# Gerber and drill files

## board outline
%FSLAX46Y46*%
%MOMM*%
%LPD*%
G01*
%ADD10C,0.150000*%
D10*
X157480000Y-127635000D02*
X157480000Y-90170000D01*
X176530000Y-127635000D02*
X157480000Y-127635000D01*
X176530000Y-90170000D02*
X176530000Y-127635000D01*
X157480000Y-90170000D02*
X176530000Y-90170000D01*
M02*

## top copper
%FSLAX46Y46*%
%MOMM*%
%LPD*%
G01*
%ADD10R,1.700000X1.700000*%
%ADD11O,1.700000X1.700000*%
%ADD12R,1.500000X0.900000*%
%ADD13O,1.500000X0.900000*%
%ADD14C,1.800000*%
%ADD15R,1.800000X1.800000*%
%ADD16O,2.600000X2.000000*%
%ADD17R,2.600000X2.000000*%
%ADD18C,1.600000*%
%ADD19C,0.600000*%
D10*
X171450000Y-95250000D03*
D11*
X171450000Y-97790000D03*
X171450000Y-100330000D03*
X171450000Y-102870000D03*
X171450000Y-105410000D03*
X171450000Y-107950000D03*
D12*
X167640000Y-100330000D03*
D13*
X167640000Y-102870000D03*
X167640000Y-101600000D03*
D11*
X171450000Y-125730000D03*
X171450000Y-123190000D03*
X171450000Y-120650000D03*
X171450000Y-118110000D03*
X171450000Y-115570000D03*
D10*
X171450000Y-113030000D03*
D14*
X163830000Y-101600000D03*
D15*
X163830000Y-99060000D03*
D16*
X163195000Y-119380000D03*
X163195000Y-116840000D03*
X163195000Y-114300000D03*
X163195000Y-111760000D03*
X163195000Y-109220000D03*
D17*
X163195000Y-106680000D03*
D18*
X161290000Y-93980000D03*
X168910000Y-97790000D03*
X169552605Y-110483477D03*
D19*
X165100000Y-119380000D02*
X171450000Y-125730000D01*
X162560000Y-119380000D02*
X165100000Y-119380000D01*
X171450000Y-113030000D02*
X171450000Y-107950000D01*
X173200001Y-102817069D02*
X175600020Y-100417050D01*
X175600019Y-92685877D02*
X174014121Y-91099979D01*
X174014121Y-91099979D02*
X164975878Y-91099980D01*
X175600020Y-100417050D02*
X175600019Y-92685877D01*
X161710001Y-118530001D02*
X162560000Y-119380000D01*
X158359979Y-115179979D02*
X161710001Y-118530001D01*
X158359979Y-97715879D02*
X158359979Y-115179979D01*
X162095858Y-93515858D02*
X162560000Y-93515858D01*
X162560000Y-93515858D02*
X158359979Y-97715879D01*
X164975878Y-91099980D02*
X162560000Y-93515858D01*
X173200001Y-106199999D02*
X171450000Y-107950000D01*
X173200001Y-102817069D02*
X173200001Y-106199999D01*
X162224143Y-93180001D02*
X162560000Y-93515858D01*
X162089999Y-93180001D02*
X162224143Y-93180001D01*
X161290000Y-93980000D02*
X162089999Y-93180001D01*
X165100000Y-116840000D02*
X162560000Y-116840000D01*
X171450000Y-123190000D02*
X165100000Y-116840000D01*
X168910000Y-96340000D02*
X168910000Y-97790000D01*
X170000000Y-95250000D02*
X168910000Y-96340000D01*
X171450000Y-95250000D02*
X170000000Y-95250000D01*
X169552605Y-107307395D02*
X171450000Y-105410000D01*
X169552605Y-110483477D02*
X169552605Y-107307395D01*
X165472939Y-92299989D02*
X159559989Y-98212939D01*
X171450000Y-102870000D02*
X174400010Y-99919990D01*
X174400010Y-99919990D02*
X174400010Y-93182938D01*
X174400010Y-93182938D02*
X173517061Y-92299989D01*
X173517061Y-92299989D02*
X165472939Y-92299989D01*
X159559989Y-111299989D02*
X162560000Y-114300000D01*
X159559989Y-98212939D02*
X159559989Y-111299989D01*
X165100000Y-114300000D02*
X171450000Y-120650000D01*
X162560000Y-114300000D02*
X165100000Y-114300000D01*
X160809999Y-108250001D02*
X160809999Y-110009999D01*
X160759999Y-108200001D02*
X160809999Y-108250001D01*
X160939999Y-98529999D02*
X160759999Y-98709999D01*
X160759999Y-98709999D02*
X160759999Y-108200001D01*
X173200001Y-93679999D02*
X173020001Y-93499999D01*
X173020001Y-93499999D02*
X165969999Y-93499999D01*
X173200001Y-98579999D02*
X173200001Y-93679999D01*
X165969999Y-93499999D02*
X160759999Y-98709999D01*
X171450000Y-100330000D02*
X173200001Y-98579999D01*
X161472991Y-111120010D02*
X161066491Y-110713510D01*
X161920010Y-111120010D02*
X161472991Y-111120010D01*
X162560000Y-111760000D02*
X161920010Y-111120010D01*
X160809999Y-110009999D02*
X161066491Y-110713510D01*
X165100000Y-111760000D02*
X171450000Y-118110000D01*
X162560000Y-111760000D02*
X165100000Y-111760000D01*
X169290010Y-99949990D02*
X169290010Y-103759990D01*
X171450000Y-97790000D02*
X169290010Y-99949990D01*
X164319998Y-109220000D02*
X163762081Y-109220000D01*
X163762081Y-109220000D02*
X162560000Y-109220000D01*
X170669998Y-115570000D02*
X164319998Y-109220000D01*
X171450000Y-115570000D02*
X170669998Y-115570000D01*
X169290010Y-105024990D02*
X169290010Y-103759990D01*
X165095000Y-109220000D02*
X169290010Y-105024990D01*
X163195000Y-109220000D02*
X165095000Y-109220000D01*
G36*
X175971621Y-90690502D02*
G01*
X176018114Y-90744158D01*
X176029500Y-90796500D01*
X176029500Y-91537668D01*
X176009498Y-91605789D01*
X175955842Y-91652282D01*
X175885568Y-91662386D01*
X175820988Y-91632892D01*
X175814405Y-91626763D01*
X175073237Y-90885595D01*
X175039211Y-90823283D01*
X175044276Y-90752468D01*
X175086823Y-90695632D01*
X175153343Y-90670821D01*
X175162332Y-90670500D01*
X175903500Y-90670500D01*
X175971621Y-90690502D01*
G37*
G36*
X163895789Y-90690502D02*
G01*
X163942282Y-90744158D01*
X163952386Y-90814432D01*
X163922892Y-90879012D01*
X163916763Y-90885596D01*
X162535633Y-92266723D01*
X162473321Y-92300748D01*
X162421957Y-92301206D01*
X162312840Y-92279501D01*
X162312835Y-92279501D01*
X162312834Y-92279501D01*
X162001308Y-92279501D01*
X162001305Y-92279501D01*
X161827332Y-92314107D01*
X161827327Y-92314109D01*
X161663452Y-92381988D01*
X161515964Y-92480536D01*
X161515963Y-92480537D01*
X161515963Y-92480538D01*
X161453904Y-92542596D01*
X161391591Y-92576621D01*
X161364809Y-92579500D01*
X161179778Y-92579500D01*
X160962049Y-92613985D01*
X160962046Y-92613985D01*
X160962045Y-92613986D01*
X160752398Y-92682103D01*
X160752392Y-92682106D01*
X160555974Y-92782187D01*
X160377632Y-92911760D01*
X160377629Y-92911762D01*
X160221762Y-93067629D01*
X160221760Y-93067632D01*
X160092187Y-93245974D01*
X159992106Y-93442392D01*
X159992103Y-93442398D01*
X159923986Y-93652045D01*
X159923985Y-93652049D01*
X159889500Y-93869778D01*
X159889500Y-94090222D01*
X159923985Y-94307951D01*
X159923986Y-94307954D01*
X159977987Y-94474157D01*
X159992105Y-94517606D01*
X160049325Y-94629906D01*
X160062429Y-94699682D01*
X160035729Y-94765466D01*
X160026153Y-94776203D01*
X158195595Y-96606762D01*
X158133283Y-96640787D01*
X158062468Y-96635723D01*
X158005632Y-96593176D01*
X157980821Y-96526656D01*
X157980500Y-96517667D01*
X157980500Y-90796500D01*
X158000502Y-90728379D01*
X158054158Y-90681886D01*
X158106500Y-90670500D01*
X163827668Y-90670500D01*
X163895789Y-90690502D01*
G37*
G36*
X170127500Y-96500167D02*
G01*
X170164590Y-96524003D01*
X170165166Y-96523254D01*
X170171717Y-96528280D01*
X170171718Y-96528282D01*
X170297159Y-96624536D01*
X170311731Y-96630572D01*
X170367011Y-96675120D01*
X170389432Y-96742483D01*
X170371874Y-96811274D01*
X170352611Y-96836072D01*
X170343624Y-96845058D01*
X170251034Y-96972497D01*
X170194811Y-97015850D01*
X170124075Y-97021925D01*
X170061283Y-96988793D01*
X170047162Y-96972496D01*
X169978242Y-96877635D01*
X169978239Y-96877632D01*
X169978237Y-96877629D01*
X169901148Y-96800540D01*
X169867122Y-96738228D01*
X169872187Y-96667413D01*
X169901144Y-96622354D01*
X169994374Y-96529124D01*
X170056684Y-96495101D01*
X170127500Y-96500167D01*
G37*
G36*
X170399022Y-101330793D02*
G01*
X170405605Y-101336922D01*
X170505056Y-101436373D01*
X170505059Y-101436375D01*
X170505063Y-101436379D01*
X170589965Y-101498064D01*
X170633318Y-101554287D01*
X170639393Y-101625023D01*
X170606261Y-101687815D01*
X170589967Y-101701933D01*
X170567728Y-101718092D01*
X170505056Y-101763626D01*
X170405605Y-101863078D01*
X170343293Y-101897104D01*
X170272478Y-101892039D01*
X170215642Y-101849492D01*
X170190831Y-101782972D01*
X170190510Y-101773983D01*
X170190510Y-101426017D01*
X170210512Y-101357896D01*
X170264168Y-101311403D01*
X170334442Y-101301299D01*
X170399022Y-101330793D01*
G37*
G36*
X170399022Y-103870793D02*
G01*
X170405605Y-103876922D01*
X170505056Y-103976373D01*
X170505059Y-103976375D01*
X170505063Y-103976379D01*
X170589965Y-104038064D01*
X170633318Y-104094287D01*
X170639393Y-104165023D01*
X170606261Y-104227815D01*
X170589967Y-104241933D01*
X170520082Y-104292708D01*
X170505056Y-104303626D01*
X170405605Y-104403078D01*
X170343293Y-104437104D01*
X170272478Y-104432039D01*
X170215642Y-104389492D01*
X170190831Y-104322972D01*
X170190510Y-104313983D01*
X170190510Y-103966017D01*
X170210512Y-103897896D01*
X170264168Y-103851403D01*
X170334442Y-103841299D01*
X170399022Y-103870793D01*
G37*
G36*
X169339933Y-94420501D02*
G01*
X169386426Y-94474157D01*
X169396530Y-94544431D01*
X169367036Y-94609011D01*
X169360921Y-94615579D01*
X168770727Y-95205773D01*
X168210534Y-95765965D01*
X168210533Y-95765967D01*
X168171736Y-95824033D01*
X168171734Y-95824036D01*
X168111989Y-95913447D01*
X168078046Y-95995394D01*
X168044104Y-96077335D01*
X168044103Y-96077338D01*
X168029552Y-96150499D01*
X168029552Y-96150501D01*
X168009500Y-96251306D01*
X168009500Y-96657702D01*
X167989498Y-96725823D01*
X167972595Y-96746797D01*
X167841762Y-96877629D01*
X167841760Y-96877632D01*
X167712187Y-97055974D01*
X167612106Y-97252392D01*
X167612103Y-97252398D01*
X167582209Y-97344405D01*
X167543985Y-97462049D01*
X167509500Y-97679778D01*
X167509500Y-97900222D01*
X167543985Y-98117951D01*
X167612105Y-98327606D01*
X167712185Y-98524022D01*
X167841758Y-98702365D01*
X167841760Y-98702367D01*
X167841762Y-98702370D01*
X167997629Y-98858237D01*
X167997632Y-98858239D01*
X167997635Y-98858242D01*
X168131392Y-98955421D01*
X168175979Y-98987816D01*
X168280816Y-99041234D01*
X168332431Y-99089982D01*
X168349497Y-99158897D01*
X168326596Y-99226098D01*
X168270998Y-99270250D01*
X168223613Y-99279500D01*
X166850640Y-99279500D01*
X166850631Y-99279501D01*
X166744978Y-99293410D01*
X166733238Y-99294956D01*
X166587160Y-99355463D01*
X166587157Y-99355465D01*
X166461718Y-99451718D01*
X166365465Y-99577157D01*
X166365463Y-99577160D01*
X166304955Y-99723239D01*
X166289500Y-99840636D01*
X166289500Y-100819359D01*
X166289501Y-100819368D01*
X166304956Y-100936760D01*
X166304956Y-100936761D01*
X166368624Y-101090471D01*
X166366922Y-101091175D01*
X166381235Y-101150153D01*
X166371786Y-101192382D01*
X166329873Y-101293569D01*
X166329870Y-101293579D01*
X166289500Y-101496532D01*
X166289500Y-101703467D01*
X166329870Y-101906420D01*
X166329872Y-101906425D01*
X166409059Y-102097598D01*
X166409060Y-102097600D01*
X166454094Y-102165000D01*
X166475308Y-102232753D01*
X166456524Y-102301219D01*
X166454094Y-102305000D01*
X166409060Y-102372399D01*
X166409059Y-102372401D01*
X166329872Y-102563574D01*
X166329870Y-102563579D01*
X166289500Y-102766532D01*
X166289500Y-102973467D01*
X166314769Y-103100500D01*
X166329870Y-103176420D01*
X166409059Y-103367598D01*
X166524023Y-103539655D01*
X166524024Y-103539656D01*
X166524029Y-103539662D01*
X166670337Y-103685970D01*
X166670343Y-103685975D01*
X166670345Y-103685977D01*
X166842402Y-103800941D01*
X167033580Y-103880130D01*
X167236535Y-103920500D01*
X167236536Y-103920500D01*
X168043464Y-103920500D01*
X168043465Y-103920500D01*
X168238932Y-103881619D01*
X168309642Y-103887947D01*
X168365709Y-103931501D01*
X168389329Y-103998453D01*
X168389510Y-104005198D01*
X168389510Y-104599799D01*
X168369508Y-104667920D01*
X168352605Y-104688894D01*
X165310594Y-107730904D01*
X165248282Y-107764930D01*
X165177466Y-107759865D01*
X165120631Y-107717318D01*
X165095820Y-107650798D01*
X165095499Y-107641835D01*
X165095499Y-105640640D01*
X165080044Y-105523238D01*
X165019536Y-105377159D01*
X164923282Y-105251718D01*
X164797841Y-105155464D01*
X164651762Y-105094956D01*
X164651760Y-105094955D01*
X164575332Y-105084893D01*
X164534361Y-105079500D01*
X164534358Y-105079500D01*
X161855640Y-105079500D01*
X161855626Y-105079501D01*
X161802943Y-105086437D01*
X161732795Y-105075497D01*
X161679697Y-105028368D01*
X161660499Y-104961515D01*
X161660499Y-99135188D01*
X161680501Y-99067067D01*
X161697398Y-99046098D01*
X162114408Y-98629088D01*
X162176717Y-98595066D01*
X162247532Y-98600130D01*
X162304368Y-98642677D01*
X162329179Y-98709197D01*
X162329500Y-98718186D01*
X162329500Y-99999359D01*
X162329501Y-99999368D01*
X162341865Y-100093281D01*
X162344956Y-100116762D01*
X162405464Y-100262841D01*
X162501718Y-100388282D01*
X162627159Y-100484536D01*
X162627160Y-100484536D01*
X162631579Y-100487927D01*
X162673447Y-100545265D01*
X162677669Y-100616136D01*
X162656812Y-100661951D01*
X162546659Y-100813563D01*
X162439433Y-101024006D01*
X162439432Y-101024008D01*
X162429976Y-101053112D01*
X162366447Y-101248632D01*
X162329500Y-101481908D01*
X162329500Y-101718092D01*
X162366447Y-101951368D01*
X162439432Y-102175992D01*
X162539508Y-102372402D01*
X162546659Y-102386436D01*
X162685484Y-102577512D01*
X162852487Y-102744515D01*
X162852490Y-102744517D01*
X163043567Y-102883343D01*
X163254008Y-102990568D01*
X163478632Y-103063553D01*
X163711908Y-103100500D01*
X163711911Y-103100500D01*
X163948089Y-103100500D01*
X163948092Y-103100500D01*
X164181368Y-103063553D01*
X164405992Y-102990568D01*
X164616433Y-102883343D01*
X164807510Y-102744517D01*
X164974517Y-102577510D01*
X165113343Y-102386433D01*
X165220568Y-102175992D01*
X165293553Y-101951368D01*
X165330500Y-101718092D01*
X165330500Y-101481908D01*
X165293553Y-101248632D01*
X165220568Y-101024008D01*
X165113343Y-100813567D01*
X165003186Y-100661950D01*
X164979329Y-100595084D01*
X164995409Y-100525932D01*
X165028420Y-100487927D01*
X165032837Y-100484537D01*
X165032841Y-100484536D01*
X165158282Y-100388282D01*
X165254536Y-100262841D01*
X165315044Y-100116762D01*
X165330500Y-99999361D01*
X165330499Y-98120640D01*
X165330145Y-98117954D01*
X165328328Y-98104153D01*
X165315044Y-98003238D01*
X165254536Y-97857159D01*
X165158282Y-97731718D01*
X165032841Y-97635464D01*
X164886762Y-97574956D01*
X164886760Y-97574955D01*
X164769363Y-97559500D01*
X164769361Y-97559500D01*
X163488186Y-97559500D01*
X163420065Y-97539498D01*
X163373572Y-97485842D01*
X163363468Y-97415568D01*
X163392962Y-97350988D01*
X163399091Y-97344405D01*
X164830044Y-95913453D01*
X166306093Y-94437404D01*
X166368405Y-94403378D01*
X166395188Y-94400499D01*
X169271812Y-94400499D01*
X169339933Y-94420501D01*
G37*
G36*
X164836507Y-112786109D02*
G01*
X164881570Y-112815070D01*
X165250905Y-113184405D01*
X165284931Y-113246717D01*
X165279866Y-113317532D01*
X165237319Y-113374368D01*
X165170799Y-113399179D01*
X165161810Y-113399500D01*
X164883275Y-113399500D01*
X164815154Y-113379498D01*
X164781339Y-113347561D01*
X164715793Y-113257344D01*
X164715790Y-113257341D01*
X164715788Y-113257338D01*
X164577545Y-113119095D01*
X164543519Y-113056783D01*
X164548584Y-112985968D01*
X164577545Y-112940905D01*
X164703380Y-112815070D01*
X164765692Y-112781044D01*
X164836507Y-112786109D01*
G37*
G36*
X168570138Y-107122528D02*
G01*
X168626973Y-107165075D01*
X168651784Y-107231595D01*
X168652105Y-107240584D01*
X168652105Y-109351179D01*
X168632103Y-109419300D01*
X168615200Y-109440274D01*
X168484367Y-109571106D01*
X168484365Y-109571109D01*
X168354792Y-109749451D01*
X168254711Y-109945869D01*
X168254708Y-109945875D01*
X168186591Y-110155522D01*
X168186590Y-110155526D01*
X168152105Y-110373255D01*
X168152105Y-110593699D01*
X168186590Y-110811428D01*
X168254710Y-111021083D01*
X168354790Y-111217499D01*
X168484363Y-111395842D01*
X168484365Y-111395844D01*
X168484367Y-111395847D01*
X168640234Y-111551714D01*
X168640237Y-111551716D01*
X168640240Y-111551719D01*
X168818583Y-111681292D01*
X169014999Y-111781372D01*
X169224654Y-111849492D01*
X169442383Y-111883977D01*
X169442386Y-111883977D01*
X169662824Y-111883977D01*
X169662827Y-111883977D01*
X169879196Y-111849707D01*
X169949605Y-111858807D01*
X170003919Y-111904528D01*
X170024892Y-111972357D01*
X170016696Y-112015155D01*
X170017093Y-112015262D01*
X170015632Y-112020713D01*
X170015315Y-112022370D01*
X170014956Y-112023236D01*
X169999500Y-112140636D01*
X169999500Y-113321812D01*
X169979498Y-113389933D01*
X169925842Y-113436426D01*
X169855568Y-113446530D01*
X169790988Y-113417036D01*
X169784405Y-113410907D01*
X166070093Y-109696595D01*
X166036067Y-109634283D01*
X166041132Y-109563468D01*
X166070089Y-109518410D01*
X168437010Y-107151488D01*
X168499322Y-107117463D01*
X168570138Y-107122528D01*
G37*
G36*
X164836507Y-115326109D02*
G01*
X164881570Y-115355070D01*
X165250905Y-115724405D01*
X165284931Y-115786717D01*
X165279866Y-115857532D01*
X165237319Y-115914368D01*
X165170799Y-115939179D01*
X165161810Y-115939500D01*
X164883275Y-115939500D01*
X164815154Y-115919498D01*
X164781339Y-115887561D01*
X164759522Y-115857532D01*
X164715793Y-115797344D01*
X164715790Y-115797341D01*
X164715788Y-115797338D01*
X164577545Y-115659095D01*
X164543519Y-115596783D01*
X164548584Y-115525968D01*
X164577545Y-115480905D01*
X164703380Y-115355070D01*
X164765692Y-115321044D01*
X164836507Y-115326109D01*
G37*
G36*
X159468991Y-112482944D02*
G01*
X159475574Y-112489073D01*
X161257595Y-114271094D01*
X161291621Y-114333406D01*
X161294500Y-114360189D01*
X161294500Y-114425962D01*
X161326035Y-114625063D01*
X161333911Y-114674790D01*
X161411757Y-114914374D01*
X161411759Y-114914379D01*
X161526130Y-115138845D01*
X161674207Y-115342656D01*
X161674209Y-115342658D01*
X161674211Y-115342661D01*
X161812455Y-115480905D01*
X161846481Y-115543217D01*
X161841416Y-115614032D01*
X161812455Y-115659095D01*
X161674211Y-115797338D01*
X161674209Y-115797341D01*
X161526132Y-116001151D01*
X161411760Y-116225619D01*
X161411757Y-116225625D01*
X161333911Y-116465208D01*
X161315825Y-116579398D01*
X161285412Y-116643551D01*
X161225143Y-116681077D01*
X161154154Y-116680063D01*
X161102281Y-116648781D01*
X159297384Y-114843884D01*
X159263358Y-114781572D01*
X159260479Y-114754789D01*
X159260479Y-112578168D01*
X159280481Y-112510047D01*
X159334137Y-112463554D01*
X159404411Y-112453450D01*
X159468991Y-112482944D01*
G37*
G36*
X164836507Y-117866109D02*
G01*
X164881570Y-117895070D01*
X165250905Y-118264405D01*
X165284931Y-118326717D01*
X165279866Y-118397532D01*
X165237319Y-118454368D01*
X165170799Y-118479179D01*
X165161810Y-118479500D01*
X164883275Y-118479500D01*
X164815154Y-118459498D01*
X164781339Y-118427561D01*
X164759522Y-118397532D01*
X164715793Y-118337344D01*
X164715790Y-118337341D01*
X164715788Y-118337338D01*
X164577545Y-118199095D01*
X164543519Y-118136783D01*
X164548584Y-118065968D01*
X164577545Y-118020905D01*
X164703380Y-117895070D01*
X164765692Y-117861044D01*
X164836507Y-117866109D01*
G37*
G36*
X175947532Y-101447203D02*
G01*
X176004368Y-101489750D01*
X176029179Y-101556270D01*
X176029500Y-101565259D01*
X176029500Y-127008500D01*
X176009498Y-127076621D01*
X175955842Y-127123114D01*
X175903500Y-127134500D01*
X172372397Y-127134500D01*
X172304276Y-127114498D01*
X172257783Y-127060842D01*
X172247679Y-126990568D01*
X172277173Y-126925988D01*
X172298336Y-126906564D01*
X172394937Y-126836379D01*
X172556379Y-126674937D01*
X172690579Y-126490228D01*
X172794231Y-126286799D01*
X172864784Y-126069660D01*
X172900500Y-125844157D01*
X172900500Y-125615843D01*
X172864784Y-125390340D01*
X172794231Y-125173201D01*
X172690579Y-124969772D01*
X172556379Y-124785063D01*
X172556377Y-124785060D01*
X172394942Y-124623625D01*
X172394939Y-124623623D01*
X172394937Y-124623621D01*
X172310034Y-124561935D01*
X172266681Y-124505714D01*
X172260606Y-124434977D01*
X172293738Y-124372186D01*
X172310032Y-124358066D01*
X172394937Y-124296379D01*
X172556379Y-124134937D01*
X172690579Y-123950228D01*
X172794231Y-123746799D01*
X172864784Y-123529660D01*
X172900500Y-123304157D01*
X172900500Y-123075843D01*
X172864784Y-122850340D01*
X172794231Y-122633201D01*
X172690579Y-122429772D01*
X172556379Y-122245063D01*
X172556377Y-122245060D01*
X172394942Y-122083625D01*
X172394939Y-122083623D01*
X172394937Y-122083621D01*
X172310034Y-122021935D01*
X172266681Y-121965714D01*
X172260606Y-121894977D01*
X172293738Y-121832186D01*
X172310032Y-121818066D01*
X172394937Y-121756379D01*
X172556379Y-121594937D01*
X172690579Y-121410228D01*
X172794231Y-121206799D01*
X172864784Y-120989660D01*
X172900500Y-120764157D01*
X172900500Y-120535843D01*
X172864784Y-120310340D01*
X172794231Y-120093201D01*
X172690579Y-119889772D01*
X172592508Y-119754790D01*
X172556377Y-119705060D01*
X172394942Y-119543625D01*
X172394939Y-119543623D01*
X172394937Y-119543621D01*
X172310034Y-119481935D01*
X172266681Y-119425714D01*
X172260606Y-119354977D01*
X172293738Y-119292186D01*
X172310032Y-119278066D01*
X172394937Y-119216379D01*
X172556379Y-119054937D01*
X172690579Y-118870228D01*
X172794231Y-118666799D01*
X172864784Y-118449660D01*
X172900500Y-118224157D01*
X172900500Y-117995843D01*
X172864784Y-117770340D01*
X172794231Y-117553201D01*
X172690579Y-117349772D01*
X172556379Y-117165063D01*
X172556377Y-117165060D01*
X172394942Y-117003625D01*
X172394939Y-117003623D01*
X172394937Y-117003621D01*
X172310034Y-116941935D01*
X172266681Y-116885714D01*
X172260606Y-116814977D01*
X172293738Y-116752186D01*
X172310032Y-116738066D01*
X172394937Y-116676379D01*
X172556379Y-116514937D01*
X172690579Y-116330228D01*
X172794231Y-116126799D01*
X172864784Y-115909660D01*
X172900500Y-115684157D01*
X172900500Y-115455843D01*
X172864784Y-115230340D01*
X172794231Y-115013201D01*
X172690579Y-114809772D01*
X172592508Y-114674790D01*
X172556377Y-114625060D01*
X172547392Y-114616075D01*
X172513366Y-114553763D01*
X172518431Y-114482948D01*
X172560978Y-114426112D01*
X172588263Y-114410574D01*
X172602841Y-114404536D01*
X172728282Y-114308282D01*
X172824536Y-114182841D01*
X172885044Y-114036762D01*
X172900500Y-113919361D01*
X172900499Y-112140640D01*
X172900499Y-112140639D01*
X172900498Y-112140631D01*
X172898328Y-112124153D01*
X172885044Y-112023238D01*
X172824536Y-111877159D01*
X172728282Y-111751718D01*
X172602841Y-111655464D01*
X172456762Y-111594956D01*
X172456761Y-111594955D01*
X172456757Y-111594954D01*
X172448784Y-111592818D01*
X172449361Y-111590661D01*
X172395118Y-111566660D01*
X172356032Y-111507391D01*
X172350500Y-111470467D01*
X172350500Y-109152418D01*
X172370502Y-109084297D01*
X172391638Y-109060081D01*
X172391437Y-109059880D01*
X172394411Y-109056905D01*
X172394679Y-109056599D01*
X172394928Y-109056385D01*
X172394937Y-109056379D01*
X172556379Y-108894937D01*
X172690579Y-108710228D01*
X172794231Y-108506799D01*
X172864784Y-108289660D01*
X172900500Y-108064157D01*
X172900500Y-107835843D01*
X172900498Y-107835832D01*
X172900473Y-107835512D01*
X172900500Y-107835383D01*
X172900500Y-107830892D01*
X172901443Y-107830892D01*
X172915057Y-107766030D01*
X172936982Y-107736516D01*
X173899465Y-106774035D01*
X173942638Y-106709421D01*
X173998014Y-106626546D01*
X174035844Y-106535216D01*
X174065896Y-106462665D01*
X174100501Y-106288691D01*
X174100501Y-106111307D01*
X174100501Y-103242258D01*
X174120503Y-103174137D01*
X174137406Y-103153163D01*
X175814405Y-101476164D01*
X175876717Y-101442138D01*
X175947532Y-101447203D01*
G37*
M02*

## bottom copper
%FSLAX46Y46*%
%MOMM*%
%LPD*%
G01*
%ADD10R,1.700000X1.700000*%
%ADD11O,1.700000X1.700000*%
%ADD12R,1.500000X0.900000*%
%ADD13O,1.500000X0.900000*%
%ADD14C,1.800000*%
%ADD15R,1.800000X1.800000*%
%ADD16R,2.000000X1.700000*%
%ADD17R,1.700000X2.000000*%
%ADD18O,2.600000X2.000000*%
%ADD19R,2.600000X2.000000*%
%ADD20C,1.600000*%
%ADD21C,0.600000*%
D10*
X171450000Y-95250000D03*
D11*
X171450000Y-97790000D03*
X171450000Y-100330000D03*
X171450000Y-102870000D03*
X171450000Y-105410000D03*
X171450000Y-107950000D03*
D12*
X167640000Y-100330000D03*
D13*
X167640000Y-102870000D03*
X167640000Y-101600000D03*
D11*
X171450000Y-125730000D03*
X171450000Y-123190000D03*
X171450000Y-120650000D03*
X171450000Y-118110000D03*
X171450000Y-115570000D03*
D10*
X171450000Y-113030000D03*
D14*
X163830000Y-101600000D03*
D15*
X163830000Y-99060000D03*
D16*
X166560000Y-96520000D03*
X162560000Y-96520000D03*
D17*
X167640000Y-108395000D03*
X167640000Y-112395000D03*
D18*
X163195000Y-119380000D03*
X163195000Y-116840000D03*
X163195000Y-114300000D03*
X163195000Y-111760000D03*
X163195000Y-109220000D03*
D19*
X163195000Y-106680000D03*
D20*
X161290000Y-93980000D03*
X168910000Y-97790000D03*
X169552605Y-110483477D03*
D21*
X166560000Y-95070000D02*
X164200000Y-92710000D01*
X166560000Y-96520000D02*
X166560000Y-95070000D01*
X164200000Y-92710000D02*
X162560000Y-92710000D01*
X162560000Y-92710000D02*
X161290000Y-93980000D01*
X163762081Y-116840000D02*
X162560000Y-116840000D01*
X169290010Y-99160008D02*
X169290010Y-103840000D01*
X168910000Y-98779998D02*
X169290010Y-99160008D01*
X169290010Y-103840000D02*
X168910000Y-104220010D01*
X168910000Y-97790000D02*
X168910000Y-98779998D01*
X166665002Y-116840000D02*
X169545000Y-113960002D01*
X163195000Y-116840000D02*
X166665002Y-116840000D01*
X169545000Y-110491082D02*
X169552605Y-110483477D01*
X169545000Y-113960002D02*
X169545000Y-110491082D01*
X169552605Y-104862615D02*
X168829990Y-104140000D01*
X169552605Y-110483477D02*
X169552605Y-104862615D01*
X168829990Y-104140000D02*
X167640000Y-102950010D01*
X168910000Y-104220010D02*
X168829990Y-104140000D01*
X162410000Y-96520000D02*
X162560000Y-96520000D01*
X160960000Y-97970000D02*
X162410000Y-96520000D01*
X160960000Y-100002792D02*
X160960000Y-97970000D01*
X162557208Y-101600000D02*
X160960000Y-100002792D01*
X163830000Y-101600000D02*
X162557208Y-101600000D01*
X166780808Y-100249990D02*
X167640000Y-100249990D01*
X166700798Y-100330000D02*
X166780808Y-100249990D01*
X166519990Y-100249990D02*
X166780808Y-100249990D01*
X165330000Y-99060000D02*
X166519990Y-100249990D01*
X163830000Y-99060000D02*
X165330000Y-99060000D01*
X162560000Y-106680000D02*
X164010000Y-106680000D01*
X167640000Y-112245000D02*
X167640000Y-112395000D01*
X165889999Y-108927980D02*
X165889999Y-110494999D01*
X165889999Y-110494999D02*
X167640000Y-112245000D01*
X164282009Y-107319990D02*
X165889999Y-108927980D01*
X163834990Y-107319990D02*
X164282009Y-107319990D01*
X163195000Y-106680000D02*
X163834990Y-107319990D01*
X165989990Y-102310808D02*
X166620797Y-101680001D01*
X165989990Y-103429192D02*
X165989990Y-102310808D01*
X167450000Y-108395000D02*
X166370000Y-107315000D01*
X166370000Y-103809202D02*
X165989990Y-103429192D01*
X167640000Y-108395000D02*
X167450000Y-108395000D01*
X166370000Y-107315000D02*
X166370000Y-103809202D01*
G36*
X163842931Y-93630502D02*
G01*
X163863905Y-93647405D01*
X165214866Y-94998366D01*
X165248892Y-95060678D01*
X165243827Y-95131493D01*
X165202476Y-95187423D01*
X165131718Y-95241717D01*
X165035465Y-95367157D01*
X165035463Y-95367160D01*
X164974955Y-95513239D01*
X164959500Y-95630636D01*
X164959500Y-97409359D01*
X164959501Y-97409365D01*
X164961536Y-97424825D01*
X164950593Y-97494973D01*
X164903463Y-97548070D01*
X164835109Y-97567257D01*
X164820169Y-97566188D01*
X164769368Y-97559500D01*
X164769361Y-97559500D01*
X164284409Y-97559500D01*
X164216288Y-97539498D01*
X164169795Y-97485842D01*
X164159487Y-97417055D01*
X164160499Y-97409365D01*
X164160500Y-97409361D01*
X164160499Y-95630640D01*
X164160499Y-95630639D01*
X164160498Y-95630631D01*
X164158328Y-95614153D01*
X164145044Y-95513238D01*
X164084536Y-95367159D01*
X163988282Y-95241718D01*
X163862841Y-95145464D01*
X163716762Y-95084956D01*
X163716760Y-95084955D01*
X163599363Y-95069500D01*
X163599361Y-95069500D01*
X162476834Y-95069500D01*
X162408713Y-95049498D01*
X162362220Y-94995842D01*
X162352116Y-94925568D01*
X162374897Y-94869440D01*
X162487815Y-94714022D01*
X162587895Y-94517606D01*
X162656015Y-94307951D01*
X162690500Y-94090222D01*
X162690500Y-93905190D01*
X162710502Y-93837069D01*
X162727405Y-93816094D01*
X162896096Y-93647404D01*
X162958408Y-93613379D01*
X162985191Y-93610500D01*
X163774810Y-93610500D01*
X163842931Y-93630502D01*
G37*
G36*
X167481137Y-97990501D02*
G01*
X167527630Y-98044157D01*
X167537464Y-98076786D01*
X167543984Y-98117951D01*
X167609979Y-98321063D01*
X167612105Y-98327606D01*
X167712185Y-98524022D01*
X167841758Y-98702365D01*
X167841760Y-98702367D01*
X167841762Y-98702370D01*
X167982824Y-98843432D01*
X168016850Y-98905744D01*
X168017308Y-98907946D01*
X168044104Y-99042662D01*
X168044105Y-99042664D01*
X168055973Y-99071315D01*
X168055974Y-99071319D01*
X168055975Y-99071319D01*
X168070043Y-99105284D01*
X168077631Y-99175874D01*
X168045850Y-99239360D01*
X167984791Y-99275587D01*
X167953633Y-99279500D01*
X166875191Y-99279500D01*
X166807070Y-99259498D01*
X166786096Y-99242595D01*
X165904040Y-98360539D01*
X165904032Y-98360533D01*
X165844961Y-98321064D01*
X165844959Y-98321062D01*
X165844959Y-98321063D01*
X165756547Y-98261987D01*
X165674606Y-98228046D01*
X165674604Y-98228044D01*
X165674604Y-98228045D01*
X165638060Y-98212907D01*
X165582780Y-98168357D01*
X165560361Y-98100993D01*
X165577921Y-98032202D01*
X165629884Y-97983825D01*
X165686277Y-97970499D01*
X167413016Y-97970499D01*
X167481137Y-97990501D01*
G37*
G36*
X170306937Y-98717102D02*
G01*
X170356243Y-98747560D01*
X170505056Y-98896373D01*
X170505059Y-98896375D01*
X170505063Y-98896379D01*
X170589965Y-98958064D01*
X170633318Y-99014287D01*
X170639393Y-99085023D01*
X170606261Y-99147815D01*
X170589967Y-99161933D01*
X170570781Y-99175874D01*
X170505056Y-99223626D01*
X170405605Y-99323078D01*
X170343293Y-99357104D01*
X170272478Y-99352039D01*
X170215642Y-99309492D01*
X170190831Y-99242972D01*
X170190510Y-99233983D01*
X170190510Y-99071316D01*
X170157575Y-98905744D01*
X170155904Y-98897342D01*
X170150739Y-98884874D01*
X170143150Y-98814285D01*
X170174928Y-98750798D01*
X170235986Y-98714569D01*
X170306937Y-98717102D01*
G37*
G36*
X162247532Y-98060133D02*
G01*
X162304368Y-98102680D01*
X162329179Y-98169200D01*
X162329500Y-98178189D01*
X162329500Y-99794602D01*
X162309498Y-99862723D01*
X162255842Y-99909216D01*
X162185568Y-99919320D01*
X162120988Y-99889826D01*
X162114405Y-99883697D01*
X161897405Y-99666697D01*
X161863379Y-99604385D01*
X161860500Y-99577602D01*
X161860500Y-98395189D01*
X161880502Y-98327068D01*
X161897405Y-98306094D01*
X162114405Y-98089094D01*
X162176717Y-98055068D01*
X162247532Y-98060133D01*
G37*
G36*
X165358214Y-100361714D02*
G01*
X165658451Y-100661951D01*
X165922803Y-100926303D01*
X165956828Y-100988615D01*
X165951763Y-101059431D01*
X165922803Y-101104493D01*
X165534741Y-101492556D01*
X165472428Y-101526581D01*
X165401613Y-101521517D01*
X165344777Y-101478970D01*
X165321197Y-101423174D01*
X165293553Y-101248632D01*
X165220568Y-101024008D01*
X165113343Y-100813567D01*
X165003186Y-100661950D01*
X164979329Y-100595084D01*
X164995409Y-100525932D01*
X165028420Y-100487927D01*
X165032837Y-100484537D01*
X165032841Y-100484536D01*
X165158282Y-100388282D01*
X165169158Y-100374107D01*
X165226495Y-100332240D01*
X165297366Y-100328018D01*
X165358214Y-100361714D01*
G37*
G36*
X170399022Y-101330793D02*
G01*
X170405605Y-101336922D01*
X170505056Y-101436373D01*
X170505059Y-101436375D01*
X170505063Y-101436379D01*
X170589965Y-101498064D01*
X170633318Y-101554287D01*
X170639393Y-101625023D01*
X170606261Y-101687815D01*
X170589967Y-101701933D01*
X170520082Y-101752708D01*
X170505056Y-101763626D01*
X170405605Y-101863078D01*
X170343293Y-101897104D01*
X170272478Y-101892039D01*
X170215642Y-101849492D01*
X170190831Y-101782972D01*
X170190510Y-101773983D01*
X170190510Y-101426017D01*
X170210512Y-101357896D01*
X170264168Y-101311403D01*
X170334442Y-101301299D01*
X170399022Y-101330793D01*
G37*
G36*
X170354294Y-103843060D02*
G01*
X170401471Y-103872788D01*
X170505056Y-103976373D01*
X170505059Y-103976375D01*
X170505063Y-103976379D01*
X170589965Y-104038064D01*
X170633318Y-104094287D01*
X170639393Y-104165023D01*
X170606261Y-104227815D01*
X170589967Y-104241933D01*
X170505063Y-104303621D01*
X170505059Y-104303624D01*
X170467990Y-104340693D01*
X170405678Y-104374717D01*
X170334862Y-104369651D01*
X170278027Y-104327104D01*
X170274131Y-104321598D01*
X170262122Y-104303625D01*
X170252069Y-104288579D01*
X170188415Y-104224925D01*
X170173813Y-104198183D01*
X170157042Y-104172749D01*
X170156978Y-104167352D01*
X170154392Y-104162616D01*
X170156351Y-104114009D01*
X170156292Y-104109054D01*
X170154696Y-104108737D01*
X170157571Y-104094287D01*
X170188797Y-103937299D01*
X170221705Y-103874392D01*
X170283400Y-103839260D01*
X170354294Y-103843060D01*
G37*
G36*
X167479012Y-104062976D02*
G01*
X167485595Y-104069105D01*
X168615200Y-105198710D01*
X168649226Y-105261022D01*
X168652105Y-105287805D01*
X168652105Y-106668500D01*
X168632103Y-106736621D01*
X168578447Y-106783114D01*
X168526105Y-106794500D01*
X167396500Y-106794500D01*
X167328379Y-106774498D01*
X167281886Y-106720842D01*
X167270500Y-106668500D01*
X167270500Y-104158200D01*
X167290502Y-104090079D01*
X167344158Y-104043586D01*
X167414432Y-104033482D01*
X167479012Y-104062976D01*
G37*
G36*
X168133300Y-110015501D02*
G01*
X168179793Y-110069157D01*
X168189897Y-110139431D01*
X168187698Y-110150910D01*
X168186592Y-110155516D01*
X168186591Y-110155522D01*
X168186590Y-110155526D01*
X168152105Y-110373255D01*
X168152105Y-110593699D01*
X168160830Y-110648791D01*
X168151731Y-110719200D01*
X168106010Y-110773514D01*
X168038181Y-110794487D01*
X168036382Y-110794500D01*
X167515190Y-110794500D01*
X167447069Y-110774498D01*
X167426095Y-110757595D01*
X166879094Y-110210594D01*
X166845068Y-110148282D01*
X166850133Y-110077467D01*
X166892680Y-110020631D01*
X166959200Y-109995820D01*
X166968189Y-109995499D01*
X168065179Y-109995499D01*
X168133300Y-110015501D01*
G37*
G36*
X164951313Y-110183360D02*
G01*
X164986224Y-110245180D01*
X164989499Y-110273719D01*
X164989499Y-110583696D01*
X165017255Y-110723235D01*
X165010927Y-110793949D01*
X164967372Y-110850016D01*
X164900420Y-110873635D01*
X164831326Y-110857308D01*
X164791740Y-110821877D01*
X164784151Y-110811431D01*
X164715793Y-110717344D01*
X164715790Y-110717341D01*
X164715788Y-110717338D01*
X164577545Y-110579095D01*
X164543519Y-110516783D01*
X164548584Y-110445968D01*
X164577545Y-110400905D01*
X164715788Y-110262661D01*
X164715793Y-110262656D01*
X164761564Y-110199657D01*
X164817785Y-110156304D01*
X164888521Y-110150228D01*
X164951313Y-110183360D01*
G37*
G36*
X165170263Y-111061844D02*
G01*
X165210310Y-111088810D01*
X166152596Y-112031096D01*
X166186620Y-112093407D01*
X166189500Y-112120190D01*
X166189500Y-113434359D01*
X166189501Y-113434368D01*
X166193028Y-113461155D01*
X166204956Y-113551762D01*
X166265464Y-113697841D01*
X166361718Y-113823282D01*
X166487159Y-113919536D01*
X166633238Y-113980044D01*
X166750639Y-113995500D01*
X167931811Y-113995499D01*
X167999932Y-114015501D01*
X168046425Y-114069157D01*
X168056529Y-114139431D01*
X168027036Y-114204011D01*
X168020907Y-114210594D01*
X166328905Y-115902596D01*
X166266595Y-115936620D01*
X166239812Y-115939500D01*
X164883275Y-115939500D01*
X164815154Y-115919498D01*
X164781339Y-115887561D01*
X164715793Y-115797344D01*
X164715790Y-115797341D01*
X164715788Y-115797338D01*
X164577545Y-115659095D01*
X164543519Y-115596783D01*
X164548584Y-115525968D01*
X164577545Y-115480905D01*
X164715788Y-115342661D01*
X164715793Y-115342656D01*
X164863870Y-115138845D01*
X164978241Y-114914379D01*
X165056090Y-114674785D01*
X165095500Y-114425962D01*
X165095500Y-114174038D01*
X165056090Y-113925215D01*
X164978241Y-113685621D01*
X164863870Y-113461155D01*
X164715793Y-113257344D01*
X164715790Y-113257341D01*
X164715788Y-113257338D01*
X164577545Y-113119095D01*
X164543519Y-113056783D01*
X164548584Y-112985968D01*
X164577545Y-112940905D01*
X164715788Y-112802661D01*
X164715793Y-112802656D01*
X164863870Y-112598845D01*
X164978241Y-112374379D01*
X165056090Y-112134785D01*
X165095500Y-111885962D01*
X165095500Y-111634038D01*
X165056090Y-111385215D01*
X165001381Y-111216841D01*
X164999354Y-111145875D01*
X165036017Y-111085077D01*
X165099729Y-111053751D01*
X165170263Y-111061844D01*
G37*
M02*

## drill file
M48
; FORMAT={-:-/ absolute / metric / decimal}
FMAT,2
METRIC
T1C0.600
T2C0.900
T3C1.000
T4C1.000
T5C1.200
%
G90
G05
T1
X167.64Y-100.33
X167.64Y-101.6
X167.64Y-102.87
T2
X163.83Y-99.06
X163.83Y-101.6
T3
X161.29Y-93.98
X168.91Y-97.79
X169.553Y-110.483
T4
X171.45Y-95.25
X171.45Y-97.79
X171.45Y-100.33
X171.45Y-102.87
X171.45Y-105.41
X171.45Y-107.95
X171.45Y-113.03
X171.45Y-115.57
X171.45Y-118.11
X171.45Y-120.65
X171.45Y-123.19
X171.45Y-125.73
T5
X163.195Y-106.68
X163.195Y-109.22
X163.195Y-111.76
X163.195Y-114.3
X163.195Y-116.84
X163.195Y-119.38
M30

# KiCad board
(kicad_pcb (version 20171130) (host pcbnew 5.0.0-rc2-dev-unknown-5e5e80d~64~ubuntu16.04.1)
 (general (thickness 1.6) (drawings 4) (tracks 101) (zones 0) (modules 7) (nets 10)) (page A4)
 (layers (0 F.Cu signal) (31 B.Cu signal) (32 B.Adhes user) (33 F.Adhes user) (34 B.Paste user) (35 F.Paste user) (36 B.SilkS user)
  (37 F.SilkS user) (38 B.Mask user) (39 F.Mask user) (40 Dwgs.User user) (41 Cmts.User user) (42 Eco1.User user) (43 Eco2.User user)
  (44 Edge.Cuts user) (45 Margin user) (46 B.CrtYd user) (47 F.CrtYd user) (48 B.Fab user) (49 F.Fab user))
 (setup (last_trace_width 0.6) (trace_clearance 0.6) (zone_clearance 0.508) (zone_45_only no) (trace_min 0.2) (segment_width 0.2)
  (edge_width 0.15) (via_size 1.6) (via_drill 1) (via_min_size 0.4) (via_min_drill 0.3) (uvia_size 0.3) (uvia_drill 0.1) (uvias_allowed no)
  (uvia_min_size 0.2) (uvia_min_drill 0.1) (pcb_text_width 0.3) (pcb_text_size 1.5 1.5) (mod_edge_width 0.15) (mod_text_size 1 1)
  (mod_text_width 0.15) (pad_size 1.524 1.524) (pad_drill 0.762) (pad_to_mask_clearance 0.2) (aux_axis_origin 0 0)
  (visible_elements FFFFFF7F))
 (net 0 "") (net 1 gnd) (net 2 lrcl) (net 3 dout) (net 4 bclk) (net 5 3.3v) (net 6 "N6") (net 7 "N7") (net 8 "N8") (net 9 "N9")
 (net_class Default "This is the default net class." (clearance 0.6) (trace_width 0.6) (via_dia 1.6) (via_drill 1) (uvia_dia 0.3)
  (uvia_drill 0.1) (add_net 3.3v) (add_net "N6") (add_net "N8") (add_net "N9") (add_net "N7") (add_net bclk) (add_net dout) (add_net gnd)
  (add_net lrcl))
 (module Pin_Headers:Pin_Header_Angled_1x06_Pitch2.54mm (layer F.Cu) (at 171.45 95.25)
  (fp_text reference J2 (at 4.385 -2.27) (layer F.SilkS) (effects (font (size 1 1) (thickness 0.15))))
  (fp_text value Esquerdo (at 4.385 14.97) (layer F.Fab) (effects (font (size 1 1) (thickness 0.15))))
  (pad 1 thru_hole rect (at 0 0) (size 1.7 1.7) (drill 1) (layers *.Cu *.Mask) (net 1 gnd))
  (pad 2 thru_hole oval (at 0 2.54) (size 1.7 1.7) (drill 1) (layers *.Cu *.Mask) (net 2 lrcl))
  (pad 3 thru_hole oval (at 0 5.08) (size 1.7 1.7) (drill 1) (layers *.Cu *.Mask) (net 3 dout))
  (pad 4 thru_hole oval (at 0 7.62) (size 1.7 1.7) (drill 1) (layers *.Cu *.Mask) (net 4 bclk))
  (pad 5 thru_hole oval (at 0 10.16) (size 1.7 1.7) (drill 1) (layers *.Cu *.Mask) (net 1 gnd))
  (pad 6 thru_hole oval (at 0 12.7) (size 1.7 1.7) (drill 1) (layers *.Cu *.Mask) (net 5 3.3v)))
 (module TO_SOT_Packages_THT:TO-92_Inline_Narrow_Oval (layer F.Cu) (at 167.64 100.33 270)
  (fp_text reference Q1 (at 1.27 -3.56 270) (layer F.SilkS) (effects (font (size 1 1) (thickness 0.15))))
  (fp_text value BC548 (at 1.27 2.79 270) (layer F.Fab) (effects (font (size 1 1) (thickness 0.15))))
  (pad 1 thru_hole rect (at 0 0 90) (size 0.9 1.5) (drill 0.6) (layers *.Cu *.Mask) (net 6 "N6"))
  (pad 3 thru_hole oval (at 2.54 0 90) (size 0.9 1.5) (drill 0.6) (layers *.Cu *.Mask) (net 1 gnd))
  (pad 2 thru_hole oval (at 1.27 0 90) (size 0.9 1.5) (drill 0.6) (layers *.Cu *.Mask) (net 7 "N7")))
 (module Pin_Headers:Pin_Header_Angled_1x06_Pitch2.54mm (layer F.Cu) (at 171.45 113.03)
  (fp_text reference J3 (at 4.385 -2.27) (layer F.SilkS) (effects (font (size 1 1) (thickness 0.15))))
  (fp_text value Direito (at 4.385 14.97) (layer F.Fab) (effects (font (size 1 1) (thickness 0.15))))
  (pad 6 thru_hole oval (at 0 12.7) (size 1.7 1.7) (drill 1) (layers *.Cu *.Mask) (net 5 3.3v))
  (pad 5 thru_hole oval (at 0 10.16) (size 1.7 1.7) (drill 1) (layers *.Cu *.Mask) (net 1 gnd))
  (pad 4 thru_hole oval (at 0 7.62) (size 1.7 1.7) (drill 1) (layers *.Cu *.Mask) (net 4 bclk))
  (pad 3 thru_hole oval (at 0 5.08) (size 1.7 1.7) (drill 1) (layers *.Cu *.Mask) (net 3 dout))
  (pad 2 thru_hole oval (at 0 2.54) (size 1.7 1.7) (drill 1) (layers *.Cu *.Mask) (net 2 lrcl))
  (pad 1 thru_hole rect (at 0 0) (size 1.7 1.7) (drill 1) (layers *.Cu *.Mask) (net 5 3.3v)))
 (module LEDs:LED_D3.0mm (layer F.Cu) (at 163.83 99.06 270)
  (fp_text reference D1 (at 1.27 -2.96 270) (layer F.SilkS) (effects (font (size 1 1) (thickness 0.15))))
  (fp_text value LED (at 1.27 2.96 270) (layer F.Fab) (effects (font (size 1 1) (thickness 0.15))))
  (pad 2 thru_hole circle (at 2.54 0 270) (size 1.8 1.8) (drill 0.9) (layers *.Cu *.Mask) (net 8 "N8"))
  (pad 1 thru_hole rect (at 0 0 270) (size 1.8 1.8) (drill 0.9) (layers *.Cu *.Mask) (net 6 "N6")))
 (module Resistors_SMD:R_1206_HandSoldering (layer B.Cu) (at 164.56 96.52)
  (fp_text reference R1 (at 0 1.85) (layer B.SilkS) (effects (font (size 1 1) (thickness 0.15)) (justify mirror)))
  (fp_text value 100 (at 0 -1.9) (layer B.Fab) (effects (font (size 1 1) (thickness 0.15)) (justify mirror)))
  (pad 2 smd rect (at 2 0) (size 2 1.7) (layers B.Cu B.Paste B.Mask) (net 5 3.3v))
  (pad 1 smd rect (at -2 0) (size 2 1.7) (layers B.Cu B.Paste B.Mask) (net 8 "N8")))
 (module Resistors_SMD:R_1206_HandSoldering (layer B.Cu) (at 167.64 110.395 270)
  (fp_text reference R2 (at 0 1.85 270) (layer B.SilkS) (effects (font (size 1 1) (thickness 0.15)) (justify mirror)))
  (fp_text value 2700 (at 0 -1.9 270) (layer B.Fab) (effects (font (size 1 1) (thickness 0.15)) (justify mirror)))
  (pad 1 smd rect (at -2 0 270) (size 2 1.7) (layers B.Cu B.Paste B.Mask) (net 7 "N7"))
  (pad 2 smd rect (at 2 0 270) (size 2 1.7) (layers B.Cu B.Paste B.Mask) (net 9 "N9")))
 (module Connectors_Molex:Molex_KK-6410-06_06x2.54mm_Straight (layer F.Cu) (at 163.195 106.68 270)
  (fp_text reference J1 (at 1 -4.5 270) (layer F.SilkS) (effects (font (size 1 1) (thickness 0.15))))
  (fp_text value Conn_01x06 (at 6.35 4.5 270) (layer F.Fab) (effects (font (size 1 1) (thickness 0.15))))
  (pad 6 thru_hole oval (at 12.7 0 270) (size 2 2.6) (drill 1.2) (layers *.Cu *.Mask) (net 5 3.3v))
  (pad 5 thru_hole oval (at 10.16 0 270) (size 2 2.6) (drill 1.2) (layers *.Cu *.Mask) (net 1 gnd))
  (pad 4 thru_hole oval (at 7.62 0 270) (size 2 2.6) (drill 1.2) (layers *.Cu *.Mask) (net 4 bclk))
  (pad 3 thru_hole oval (at 5.08 0 270) (size 2 2.6) (drill 1.2) (layers *.Cu *.Mask) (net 3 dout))
  (pad 2 thru_hole oval (at 2.54 0 270) (size 2 2.6) (drill 1.2) (layers *.Cu *.Mask) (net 2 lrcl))
  (pad 1 thru_hole rect (at 0 0 270) (size 2 2.6) (drill 1.2) (layers *.Cu *.Mask) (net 9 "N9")))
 (gr_line (start 157.48 127.635) (end 157.48 90.17) (layer Edge.Cuts) (width 0.15))
 (gr_line (start 176.53 127.635) (end 157.48 127.635) (layer Edge.Cuts) (width 0.15))
 (gr_line (start 176.53 90.17) (end 176.53 127.635) (layer Edge.Cuts) (width 0.15))
 (gr_line (start 157.48 90.17) (end 176.53 90.17) (layer Edge.Cuts) (width 0.15))
 (segment (start 165.1 119.38) (end 171.45 125.73) (width 0.6) (layer F.Cu) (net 5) (status 20))
 (segment (start 162.56 119.38) (end 165.1 119.38) (width 0.6) (layer F.Cu) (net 5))
 (segment (start 171.45 113.03) (end 171.45 107.95) (width 0.6) (layer F.Cu) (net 5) (status 30))
 (segment (start 173.200001 102.817069) (end 175.60002 100.41705) (width 0.6) (layer F.Cu) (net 5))
 (segment (start 175.600019 92.685877) (end 174.014121 91.099979) (width 0.6) (layer F.Cu) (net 5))
 (segment (start 174.014121 91.099979) (end 164.975878 91.09998) (width 0.6) (layer F.Cu) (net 5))
 (segment (start 175.60002 100.41705) (end 175.600019 92.685877) (width 0.6) (layer F.Cu) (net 5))
 (segment (start 161.710001 118.530001) (end 162.56 119.38) (width 0.6) (layer F.Cu) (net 5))
 (segment (start 158.359979 115.179979) (end 161.710001 118.530001) (width 0.6) (layer F.Cu) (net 5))
 (segment (start 158.359979 97.715879) (end 158.359979 115.179979) (width 0.6) (layer F.Cu) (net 5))
 (segment (start 166.56 95.07) (end 164.2 92.71) (width 0.6) (layer B.Cu) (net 5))
 (segment (start 166.56 96.52) (end 166.56 95.07) (width 0.6) (layer B.Cu) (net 5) (status 10))
 (segment (start 162.095858 93.515858) (end 162.56 93.515858) (width 0.6) (layer F.Cu) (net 5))
 (segment (start 162.56 93.515858) (end 158.359979 97.715879) (width 0.6) (layer F.Cu) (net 5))
 (segment (start 164.975878 91.09998) (end 162.56 93.515858) (width 0.6) (layer F.Cu) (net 5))
 (segment (start 173.200001 106.199999) (end 171.45 107.95) (width 0.6) (layer F.Cu) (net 5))
 (segment (start 173.200001 102.817069) (end 173.200001 106.199999) (width 0.6) (layer F.Cu) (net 5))
 (segment (start 164.2 92.71) (end 162.56 92.71) (width 0.6) (layer B.Cu) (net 5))
 (segment (start 162.56 92.71) (end 161.29 93.98) (width 0.6) (layer B.Cu) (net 5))
 (via (at 161.29 93.98) (size 1.6) (drill 1) (layers F.Cu B.Cu) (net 5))
 (segment (start 162.224143 93.180001) (end 162.56 93.515858) (width 0.6) (layer F.Cu) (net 5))
 (segment (start 162.089999 93.180001) (end 162.224143 93.180001) (width 0.6) (layer F.Cu) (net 5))
 (segment (start 161.29 93.98) (end 162.089999 93.180001) (width 0.6) (layer F.Cu) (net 5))
 (segment (start 165.1 116.84) (end 162.56 116.84) (width 0.6) (layer F.Cu) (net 1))
 (segment (start 171.45 123.19) (end 165.1 116.84) (width 0.6) (layer F.Cu) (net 1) (status 10))
 (segment (start 163.762081 116.84) (end 162.56 116.84) (width 0.6) (layer B.Cu) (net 1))
 (segment (start 168.91 96.34) (end 168.91 97.79) (width 0.6) (layer F.Cu) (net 1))
 (segment (start 169.29001 99.160008) (end 169.29001 103.84) (width 0.6) (layer B.Cu) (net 1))
 (segment (start 168.91 98.779998) (end 169.29001 99.160008) (width 0.6) (layer B.Cu) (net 1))
 (segment (start 169.29001 103.84) (end 168.91 104.22001) (width 0.6) (layer B.Cu) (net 1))
 (segment (start 168.91 97.79) (end 168.91 98.779998) (width 0.6) (layer B.Cu) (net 1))
 (segment (start 170 95.25) (end 168.91 96.34) (width 0.6) (layer F.Cu) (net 1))
 (segment (start 171.45 95.25) (end 170 95.25) (width 0.6) (layer F.Cu) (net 1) (status 10))
 (via (at 168.91 97.79) (size 1.6) (drill 1) (layers F.Cu B.Cu) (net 1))
 (segment (start 166.665002 116.84) (end 169.545 113.960002) (width 0.6) (layer B.Cu) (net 1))
 (segment (start 163.195 116.84) (end 166.665002 116.84) (width 0.6) (layer B.Cu) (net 1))
 (via (at 169.552605 110.483477) (size 1.6) (drill 1) (layers F.Cu B.Cu) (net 1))
 (segment (start 169.545 110.491082) (end 169.552605 110.483477) (width 0.6) (layer B.Cu) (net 1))
 (segment (start 169.545 113.960002) (end 169.545 110.491082) (width 0.6) (layer B.Cu) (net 1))
 (segment (start 169.552605 107.307395) (end 171.45 105.41) (width 0.6) (layer F.Cu) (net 1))
 (segment (start 169.552605 110.483477) (end 169.552605 107.307395) (width 0.6) (layer F.Cu) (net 1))
 (segment (start 169.552605 104.862615) (end 168.82999 104.14) (width 0.6) (layer B.Cu) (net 1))
 (segment (start 169.552605 110.483477) (end 169.552605 104.862615) (width 0.6) (layer B.Cu) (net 1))
 (segment (start 168.82999 104.14) (end 167.64 102.95001) (width 0.6) (layer B.Cu) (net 1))
 (segment (start 168.91 104.22001) (end 168.82999 104.14) (width 0.6) (layer B.Cu) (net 1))
 (segment (start 165.472939 92.299989) (end 159.559989 98.212939) (width 0.6) (layer F.Cu) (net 4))
 (segment (start 171.45 102.87) (end 174.40001 99.91999) (width 0.6) (layer F.Cu) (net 4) (status 10))
 (segment (start 174.40001 99.91999) (end 174.40001 93.182938) (width 0.6) (layer F.Cu) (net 4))
 (segment (start 174.40001 93.182938) (end 173.517061 92.299989) (width 0.6) (layer F.Cu) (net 4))
 (segment (start 173.517061 92.299989) (end 165.472939 92.299989) (width 0.6) (layer F.Cu) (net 4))
 (segment (start 159.559989 111.299989) (end 162.56 114.3) (width 0.6) (layer F.Cu) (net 4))
 (segment (start 159.559989 98.212939) (end 159.559989 111.299989) (width 0.6) (layer F.Cu) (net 4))
 (segment (start 165.1 114.3) (end 171.45 120.65) (width 0.6) (layer F.Cu) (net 4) (status 20))
 (segment (start 162.56 114.3) (end 165.1 114.3) (width 0.6) (layer F.Cu) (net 4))
 (segment (start 160.809999 108.250001) (end 160.809999 110.009999) (width 0.6) (layer F.Cu) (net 3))
 (segment (start 160.759999 108.200001) (end 160.809999 108.250001) (width 0.6) (layer F.Cu) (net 3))
 (segment (start 160.939999 98.529999) (end 160.759999 98.709999) (width 0.6) (layer F.Cu) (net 3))
 (segment (start 160.759999 98.709999) (end 160.759999 108.200001) (width 0.6) (layer F.Cu) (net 3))
 (segment (start 173.200001 93.679999) (end 173.020001 93.499999) (width 0.6) (layer F.Cu) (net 3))
 (segment (start 173.020001 93.499999) (end 165.969999 93.499999) (width 0.6) (layer F.Cu) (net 3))
 (segment (start 173.200001 98.579999) (end 173.200001 93.679999) (width 0.6) (layer F.Cu) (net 3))
 (segment (start 165.969999 93.499999) (end 160.759999 98.709999) (width 0.6) (layer F.Cu) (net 3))
 (segment (start 171.45 100.33) (end 173.200001 98.579999) (width 0.6) (layer F.Cu) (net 3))
 (segment (start 161.472991 111.12001) (end 161.066491 110.71351) (width 0.6) (layer F.Cu) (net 3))
 (segment (start 161.92001 111.12001) (end 161.472991 111.12001) (width 0.6) (layer F.Cu) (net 3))
 (segment (start 162.56 111.76) (end 161.92001 111.12001) (width 0.6) (layer F.Cu) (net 3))
 (segment (start 160.809999 110.009999) (end 161.066491 110.71351) (width 0.6) (layer F.Cu) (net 3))
 (segment (start 165.1 111.76) (end 171.45 118.11) (width 0.6) (layer F.Cu) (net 3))
 (segment (start 162.56 111.76) (end 165.1 111.76) (width 0.6) (layer F.Cu) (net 3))
 (segment (start 169.29001 99.94999) (end 169.29001 103.75999) (width 0.6) (layer F.Cu) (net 2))
 (segment (start 171.45 97.79) (end 169.29001 99.94999) (width 0.6) (layer F.Cu) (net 2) (status 10))
 (segment (start 164.319998 109.22) (end 163.762081 109.22) (width 0.6) (layer F.Cu) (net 2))
 (segment (start 163.762081 109.22) (end 162.56 109.22) (width 0.6) (layer F.Cu) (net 2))
 (segment (start 170.669998 115.57) (end 164.319998 109.22) (width 0.6) (layer F.Cu) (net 2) (status 10))
 (segment (start 171.45 115.57) (end 170.669998 115.57) (width 0.6) (layer F.Cu) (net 2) (status 30))
 (segment (start 169.29001 105.02499) (end 169.29001 103.75999) (width 0.6) (layer F.Cu) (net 2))
 (segment (start 165.095 109.22) (end 169.29001 105.02499) (width 0.6) (layer F.Cu) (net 2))
 (segment (start 163.195 109.22) (end 165.095 109.22) (width 0.6) (layer F.Cu) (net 2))
 (segment (start 162.41 96.52) (end 162.56 96.52) (width 0.6) (layer B.Cu) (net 8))
 (segment (start 160.96 97.97) (end 162.41 96.52) (width 0.6) (layer B.Cu) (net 8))
 (segment (start 160.96 100.002792) (end 160.96 97.97) (width 0.6) (layer B.Cu) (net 8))
 (segment (start 162.557208 101.6) (end 160.96 100.002792) (width 0.6) (layer B.Cu) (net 8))
 (segment (start 163.83 101.6) (end 162.557208 101.6) (width 0.6) (layer B.Cu) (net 8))
 (segment (start 166.780808 100.24999) (end 167.64 100.24999) (width 0.6) (layer B.Cu) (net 6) (status 20))
 (segment (start 166.700798 100.33) (end 166.780808 100.24999) (width 0.6) (layer B.Cu) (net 6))
 (segment (start 166.51999 100.24999) (end 166.780808 100.24999) (width 0.6) (layer B.Cu) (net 6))
 (segment (start 165.33 99.06) (end 166.51999 100.24999) (width 0.6) (layer B.Cu) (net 6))
 (segment (start 163.83 99.06) (end 165.33 99.06) (width 0.6) (layer B.Cu) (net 6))
 (segment (start 162.56 106.68) (end 164.01 106.68) (width 0.6) (layer B.Cu) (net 9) (status 10))
 (segment (start 167.64 112.245) (end 167.64 112.395) (width 0.6) (layer B.Cu) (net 9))
 (segment (start 165.889999 108.92798) (end 165.889999 110.494999) (width 0.6) (layer B.Cu) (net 9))
 (segment (start 165.889999 110.494999) (end 167.64 112.245) (width 0.6) (layer B.Cu) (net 9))
 (segment (start 164.282009 107.31999) (end 165.889999 108.92798) (width 0.6) (layer B.Cu) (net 9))
 (segment (start 163.83499 107.31999) (end 164.282009 107.31999) (width 0.6) (layer B.Cu) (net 9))
 (segment (start 163.195 106.68) (end 163.83499 107.31999) (width 0.6) (layer B.Cu) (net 9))
 (segment (start 165.98999 102.310808) (end 166.620797 101.680001) (width 0.6) (layer B.Cu) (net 7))
 (segment (start 165.98999 103.429192) (end 165.98999 102.310808) (width 0.6) (layer B.Cu) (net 7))
 (segment (start 167.45 108.395) (end 166.37 107.315) (width 0.6) (layer B.Cu) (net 7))
 (segment (start 166.37 103.809202) (end 165.98999 103.429192) (width 0.6) (layer B.Cu) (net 7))
 (segment (start 167.64 108.395) (end 167.45 108.395) (width 0.6) (layer B.Cu) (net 7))
 (segment (start 166.37 107.315) (end 166.37 103.809202) (width 0.6) (layer B.Cu) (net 7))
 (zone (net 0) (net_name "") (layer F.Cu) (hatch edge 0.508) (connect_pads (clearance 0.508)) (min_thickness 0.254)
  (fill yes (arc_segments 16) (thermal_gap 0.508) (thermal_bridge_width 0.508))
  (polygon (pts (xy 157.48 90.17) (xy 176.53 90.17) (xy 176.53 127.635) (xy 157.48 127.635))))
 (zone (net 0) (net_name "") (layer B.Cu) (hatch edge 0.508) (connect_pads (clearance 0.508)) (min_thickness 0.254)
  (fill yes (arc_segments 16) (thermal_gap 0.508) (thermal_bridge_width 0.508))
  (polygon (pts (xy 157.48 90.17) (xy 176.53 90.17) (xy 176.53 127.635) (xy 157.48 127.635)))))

